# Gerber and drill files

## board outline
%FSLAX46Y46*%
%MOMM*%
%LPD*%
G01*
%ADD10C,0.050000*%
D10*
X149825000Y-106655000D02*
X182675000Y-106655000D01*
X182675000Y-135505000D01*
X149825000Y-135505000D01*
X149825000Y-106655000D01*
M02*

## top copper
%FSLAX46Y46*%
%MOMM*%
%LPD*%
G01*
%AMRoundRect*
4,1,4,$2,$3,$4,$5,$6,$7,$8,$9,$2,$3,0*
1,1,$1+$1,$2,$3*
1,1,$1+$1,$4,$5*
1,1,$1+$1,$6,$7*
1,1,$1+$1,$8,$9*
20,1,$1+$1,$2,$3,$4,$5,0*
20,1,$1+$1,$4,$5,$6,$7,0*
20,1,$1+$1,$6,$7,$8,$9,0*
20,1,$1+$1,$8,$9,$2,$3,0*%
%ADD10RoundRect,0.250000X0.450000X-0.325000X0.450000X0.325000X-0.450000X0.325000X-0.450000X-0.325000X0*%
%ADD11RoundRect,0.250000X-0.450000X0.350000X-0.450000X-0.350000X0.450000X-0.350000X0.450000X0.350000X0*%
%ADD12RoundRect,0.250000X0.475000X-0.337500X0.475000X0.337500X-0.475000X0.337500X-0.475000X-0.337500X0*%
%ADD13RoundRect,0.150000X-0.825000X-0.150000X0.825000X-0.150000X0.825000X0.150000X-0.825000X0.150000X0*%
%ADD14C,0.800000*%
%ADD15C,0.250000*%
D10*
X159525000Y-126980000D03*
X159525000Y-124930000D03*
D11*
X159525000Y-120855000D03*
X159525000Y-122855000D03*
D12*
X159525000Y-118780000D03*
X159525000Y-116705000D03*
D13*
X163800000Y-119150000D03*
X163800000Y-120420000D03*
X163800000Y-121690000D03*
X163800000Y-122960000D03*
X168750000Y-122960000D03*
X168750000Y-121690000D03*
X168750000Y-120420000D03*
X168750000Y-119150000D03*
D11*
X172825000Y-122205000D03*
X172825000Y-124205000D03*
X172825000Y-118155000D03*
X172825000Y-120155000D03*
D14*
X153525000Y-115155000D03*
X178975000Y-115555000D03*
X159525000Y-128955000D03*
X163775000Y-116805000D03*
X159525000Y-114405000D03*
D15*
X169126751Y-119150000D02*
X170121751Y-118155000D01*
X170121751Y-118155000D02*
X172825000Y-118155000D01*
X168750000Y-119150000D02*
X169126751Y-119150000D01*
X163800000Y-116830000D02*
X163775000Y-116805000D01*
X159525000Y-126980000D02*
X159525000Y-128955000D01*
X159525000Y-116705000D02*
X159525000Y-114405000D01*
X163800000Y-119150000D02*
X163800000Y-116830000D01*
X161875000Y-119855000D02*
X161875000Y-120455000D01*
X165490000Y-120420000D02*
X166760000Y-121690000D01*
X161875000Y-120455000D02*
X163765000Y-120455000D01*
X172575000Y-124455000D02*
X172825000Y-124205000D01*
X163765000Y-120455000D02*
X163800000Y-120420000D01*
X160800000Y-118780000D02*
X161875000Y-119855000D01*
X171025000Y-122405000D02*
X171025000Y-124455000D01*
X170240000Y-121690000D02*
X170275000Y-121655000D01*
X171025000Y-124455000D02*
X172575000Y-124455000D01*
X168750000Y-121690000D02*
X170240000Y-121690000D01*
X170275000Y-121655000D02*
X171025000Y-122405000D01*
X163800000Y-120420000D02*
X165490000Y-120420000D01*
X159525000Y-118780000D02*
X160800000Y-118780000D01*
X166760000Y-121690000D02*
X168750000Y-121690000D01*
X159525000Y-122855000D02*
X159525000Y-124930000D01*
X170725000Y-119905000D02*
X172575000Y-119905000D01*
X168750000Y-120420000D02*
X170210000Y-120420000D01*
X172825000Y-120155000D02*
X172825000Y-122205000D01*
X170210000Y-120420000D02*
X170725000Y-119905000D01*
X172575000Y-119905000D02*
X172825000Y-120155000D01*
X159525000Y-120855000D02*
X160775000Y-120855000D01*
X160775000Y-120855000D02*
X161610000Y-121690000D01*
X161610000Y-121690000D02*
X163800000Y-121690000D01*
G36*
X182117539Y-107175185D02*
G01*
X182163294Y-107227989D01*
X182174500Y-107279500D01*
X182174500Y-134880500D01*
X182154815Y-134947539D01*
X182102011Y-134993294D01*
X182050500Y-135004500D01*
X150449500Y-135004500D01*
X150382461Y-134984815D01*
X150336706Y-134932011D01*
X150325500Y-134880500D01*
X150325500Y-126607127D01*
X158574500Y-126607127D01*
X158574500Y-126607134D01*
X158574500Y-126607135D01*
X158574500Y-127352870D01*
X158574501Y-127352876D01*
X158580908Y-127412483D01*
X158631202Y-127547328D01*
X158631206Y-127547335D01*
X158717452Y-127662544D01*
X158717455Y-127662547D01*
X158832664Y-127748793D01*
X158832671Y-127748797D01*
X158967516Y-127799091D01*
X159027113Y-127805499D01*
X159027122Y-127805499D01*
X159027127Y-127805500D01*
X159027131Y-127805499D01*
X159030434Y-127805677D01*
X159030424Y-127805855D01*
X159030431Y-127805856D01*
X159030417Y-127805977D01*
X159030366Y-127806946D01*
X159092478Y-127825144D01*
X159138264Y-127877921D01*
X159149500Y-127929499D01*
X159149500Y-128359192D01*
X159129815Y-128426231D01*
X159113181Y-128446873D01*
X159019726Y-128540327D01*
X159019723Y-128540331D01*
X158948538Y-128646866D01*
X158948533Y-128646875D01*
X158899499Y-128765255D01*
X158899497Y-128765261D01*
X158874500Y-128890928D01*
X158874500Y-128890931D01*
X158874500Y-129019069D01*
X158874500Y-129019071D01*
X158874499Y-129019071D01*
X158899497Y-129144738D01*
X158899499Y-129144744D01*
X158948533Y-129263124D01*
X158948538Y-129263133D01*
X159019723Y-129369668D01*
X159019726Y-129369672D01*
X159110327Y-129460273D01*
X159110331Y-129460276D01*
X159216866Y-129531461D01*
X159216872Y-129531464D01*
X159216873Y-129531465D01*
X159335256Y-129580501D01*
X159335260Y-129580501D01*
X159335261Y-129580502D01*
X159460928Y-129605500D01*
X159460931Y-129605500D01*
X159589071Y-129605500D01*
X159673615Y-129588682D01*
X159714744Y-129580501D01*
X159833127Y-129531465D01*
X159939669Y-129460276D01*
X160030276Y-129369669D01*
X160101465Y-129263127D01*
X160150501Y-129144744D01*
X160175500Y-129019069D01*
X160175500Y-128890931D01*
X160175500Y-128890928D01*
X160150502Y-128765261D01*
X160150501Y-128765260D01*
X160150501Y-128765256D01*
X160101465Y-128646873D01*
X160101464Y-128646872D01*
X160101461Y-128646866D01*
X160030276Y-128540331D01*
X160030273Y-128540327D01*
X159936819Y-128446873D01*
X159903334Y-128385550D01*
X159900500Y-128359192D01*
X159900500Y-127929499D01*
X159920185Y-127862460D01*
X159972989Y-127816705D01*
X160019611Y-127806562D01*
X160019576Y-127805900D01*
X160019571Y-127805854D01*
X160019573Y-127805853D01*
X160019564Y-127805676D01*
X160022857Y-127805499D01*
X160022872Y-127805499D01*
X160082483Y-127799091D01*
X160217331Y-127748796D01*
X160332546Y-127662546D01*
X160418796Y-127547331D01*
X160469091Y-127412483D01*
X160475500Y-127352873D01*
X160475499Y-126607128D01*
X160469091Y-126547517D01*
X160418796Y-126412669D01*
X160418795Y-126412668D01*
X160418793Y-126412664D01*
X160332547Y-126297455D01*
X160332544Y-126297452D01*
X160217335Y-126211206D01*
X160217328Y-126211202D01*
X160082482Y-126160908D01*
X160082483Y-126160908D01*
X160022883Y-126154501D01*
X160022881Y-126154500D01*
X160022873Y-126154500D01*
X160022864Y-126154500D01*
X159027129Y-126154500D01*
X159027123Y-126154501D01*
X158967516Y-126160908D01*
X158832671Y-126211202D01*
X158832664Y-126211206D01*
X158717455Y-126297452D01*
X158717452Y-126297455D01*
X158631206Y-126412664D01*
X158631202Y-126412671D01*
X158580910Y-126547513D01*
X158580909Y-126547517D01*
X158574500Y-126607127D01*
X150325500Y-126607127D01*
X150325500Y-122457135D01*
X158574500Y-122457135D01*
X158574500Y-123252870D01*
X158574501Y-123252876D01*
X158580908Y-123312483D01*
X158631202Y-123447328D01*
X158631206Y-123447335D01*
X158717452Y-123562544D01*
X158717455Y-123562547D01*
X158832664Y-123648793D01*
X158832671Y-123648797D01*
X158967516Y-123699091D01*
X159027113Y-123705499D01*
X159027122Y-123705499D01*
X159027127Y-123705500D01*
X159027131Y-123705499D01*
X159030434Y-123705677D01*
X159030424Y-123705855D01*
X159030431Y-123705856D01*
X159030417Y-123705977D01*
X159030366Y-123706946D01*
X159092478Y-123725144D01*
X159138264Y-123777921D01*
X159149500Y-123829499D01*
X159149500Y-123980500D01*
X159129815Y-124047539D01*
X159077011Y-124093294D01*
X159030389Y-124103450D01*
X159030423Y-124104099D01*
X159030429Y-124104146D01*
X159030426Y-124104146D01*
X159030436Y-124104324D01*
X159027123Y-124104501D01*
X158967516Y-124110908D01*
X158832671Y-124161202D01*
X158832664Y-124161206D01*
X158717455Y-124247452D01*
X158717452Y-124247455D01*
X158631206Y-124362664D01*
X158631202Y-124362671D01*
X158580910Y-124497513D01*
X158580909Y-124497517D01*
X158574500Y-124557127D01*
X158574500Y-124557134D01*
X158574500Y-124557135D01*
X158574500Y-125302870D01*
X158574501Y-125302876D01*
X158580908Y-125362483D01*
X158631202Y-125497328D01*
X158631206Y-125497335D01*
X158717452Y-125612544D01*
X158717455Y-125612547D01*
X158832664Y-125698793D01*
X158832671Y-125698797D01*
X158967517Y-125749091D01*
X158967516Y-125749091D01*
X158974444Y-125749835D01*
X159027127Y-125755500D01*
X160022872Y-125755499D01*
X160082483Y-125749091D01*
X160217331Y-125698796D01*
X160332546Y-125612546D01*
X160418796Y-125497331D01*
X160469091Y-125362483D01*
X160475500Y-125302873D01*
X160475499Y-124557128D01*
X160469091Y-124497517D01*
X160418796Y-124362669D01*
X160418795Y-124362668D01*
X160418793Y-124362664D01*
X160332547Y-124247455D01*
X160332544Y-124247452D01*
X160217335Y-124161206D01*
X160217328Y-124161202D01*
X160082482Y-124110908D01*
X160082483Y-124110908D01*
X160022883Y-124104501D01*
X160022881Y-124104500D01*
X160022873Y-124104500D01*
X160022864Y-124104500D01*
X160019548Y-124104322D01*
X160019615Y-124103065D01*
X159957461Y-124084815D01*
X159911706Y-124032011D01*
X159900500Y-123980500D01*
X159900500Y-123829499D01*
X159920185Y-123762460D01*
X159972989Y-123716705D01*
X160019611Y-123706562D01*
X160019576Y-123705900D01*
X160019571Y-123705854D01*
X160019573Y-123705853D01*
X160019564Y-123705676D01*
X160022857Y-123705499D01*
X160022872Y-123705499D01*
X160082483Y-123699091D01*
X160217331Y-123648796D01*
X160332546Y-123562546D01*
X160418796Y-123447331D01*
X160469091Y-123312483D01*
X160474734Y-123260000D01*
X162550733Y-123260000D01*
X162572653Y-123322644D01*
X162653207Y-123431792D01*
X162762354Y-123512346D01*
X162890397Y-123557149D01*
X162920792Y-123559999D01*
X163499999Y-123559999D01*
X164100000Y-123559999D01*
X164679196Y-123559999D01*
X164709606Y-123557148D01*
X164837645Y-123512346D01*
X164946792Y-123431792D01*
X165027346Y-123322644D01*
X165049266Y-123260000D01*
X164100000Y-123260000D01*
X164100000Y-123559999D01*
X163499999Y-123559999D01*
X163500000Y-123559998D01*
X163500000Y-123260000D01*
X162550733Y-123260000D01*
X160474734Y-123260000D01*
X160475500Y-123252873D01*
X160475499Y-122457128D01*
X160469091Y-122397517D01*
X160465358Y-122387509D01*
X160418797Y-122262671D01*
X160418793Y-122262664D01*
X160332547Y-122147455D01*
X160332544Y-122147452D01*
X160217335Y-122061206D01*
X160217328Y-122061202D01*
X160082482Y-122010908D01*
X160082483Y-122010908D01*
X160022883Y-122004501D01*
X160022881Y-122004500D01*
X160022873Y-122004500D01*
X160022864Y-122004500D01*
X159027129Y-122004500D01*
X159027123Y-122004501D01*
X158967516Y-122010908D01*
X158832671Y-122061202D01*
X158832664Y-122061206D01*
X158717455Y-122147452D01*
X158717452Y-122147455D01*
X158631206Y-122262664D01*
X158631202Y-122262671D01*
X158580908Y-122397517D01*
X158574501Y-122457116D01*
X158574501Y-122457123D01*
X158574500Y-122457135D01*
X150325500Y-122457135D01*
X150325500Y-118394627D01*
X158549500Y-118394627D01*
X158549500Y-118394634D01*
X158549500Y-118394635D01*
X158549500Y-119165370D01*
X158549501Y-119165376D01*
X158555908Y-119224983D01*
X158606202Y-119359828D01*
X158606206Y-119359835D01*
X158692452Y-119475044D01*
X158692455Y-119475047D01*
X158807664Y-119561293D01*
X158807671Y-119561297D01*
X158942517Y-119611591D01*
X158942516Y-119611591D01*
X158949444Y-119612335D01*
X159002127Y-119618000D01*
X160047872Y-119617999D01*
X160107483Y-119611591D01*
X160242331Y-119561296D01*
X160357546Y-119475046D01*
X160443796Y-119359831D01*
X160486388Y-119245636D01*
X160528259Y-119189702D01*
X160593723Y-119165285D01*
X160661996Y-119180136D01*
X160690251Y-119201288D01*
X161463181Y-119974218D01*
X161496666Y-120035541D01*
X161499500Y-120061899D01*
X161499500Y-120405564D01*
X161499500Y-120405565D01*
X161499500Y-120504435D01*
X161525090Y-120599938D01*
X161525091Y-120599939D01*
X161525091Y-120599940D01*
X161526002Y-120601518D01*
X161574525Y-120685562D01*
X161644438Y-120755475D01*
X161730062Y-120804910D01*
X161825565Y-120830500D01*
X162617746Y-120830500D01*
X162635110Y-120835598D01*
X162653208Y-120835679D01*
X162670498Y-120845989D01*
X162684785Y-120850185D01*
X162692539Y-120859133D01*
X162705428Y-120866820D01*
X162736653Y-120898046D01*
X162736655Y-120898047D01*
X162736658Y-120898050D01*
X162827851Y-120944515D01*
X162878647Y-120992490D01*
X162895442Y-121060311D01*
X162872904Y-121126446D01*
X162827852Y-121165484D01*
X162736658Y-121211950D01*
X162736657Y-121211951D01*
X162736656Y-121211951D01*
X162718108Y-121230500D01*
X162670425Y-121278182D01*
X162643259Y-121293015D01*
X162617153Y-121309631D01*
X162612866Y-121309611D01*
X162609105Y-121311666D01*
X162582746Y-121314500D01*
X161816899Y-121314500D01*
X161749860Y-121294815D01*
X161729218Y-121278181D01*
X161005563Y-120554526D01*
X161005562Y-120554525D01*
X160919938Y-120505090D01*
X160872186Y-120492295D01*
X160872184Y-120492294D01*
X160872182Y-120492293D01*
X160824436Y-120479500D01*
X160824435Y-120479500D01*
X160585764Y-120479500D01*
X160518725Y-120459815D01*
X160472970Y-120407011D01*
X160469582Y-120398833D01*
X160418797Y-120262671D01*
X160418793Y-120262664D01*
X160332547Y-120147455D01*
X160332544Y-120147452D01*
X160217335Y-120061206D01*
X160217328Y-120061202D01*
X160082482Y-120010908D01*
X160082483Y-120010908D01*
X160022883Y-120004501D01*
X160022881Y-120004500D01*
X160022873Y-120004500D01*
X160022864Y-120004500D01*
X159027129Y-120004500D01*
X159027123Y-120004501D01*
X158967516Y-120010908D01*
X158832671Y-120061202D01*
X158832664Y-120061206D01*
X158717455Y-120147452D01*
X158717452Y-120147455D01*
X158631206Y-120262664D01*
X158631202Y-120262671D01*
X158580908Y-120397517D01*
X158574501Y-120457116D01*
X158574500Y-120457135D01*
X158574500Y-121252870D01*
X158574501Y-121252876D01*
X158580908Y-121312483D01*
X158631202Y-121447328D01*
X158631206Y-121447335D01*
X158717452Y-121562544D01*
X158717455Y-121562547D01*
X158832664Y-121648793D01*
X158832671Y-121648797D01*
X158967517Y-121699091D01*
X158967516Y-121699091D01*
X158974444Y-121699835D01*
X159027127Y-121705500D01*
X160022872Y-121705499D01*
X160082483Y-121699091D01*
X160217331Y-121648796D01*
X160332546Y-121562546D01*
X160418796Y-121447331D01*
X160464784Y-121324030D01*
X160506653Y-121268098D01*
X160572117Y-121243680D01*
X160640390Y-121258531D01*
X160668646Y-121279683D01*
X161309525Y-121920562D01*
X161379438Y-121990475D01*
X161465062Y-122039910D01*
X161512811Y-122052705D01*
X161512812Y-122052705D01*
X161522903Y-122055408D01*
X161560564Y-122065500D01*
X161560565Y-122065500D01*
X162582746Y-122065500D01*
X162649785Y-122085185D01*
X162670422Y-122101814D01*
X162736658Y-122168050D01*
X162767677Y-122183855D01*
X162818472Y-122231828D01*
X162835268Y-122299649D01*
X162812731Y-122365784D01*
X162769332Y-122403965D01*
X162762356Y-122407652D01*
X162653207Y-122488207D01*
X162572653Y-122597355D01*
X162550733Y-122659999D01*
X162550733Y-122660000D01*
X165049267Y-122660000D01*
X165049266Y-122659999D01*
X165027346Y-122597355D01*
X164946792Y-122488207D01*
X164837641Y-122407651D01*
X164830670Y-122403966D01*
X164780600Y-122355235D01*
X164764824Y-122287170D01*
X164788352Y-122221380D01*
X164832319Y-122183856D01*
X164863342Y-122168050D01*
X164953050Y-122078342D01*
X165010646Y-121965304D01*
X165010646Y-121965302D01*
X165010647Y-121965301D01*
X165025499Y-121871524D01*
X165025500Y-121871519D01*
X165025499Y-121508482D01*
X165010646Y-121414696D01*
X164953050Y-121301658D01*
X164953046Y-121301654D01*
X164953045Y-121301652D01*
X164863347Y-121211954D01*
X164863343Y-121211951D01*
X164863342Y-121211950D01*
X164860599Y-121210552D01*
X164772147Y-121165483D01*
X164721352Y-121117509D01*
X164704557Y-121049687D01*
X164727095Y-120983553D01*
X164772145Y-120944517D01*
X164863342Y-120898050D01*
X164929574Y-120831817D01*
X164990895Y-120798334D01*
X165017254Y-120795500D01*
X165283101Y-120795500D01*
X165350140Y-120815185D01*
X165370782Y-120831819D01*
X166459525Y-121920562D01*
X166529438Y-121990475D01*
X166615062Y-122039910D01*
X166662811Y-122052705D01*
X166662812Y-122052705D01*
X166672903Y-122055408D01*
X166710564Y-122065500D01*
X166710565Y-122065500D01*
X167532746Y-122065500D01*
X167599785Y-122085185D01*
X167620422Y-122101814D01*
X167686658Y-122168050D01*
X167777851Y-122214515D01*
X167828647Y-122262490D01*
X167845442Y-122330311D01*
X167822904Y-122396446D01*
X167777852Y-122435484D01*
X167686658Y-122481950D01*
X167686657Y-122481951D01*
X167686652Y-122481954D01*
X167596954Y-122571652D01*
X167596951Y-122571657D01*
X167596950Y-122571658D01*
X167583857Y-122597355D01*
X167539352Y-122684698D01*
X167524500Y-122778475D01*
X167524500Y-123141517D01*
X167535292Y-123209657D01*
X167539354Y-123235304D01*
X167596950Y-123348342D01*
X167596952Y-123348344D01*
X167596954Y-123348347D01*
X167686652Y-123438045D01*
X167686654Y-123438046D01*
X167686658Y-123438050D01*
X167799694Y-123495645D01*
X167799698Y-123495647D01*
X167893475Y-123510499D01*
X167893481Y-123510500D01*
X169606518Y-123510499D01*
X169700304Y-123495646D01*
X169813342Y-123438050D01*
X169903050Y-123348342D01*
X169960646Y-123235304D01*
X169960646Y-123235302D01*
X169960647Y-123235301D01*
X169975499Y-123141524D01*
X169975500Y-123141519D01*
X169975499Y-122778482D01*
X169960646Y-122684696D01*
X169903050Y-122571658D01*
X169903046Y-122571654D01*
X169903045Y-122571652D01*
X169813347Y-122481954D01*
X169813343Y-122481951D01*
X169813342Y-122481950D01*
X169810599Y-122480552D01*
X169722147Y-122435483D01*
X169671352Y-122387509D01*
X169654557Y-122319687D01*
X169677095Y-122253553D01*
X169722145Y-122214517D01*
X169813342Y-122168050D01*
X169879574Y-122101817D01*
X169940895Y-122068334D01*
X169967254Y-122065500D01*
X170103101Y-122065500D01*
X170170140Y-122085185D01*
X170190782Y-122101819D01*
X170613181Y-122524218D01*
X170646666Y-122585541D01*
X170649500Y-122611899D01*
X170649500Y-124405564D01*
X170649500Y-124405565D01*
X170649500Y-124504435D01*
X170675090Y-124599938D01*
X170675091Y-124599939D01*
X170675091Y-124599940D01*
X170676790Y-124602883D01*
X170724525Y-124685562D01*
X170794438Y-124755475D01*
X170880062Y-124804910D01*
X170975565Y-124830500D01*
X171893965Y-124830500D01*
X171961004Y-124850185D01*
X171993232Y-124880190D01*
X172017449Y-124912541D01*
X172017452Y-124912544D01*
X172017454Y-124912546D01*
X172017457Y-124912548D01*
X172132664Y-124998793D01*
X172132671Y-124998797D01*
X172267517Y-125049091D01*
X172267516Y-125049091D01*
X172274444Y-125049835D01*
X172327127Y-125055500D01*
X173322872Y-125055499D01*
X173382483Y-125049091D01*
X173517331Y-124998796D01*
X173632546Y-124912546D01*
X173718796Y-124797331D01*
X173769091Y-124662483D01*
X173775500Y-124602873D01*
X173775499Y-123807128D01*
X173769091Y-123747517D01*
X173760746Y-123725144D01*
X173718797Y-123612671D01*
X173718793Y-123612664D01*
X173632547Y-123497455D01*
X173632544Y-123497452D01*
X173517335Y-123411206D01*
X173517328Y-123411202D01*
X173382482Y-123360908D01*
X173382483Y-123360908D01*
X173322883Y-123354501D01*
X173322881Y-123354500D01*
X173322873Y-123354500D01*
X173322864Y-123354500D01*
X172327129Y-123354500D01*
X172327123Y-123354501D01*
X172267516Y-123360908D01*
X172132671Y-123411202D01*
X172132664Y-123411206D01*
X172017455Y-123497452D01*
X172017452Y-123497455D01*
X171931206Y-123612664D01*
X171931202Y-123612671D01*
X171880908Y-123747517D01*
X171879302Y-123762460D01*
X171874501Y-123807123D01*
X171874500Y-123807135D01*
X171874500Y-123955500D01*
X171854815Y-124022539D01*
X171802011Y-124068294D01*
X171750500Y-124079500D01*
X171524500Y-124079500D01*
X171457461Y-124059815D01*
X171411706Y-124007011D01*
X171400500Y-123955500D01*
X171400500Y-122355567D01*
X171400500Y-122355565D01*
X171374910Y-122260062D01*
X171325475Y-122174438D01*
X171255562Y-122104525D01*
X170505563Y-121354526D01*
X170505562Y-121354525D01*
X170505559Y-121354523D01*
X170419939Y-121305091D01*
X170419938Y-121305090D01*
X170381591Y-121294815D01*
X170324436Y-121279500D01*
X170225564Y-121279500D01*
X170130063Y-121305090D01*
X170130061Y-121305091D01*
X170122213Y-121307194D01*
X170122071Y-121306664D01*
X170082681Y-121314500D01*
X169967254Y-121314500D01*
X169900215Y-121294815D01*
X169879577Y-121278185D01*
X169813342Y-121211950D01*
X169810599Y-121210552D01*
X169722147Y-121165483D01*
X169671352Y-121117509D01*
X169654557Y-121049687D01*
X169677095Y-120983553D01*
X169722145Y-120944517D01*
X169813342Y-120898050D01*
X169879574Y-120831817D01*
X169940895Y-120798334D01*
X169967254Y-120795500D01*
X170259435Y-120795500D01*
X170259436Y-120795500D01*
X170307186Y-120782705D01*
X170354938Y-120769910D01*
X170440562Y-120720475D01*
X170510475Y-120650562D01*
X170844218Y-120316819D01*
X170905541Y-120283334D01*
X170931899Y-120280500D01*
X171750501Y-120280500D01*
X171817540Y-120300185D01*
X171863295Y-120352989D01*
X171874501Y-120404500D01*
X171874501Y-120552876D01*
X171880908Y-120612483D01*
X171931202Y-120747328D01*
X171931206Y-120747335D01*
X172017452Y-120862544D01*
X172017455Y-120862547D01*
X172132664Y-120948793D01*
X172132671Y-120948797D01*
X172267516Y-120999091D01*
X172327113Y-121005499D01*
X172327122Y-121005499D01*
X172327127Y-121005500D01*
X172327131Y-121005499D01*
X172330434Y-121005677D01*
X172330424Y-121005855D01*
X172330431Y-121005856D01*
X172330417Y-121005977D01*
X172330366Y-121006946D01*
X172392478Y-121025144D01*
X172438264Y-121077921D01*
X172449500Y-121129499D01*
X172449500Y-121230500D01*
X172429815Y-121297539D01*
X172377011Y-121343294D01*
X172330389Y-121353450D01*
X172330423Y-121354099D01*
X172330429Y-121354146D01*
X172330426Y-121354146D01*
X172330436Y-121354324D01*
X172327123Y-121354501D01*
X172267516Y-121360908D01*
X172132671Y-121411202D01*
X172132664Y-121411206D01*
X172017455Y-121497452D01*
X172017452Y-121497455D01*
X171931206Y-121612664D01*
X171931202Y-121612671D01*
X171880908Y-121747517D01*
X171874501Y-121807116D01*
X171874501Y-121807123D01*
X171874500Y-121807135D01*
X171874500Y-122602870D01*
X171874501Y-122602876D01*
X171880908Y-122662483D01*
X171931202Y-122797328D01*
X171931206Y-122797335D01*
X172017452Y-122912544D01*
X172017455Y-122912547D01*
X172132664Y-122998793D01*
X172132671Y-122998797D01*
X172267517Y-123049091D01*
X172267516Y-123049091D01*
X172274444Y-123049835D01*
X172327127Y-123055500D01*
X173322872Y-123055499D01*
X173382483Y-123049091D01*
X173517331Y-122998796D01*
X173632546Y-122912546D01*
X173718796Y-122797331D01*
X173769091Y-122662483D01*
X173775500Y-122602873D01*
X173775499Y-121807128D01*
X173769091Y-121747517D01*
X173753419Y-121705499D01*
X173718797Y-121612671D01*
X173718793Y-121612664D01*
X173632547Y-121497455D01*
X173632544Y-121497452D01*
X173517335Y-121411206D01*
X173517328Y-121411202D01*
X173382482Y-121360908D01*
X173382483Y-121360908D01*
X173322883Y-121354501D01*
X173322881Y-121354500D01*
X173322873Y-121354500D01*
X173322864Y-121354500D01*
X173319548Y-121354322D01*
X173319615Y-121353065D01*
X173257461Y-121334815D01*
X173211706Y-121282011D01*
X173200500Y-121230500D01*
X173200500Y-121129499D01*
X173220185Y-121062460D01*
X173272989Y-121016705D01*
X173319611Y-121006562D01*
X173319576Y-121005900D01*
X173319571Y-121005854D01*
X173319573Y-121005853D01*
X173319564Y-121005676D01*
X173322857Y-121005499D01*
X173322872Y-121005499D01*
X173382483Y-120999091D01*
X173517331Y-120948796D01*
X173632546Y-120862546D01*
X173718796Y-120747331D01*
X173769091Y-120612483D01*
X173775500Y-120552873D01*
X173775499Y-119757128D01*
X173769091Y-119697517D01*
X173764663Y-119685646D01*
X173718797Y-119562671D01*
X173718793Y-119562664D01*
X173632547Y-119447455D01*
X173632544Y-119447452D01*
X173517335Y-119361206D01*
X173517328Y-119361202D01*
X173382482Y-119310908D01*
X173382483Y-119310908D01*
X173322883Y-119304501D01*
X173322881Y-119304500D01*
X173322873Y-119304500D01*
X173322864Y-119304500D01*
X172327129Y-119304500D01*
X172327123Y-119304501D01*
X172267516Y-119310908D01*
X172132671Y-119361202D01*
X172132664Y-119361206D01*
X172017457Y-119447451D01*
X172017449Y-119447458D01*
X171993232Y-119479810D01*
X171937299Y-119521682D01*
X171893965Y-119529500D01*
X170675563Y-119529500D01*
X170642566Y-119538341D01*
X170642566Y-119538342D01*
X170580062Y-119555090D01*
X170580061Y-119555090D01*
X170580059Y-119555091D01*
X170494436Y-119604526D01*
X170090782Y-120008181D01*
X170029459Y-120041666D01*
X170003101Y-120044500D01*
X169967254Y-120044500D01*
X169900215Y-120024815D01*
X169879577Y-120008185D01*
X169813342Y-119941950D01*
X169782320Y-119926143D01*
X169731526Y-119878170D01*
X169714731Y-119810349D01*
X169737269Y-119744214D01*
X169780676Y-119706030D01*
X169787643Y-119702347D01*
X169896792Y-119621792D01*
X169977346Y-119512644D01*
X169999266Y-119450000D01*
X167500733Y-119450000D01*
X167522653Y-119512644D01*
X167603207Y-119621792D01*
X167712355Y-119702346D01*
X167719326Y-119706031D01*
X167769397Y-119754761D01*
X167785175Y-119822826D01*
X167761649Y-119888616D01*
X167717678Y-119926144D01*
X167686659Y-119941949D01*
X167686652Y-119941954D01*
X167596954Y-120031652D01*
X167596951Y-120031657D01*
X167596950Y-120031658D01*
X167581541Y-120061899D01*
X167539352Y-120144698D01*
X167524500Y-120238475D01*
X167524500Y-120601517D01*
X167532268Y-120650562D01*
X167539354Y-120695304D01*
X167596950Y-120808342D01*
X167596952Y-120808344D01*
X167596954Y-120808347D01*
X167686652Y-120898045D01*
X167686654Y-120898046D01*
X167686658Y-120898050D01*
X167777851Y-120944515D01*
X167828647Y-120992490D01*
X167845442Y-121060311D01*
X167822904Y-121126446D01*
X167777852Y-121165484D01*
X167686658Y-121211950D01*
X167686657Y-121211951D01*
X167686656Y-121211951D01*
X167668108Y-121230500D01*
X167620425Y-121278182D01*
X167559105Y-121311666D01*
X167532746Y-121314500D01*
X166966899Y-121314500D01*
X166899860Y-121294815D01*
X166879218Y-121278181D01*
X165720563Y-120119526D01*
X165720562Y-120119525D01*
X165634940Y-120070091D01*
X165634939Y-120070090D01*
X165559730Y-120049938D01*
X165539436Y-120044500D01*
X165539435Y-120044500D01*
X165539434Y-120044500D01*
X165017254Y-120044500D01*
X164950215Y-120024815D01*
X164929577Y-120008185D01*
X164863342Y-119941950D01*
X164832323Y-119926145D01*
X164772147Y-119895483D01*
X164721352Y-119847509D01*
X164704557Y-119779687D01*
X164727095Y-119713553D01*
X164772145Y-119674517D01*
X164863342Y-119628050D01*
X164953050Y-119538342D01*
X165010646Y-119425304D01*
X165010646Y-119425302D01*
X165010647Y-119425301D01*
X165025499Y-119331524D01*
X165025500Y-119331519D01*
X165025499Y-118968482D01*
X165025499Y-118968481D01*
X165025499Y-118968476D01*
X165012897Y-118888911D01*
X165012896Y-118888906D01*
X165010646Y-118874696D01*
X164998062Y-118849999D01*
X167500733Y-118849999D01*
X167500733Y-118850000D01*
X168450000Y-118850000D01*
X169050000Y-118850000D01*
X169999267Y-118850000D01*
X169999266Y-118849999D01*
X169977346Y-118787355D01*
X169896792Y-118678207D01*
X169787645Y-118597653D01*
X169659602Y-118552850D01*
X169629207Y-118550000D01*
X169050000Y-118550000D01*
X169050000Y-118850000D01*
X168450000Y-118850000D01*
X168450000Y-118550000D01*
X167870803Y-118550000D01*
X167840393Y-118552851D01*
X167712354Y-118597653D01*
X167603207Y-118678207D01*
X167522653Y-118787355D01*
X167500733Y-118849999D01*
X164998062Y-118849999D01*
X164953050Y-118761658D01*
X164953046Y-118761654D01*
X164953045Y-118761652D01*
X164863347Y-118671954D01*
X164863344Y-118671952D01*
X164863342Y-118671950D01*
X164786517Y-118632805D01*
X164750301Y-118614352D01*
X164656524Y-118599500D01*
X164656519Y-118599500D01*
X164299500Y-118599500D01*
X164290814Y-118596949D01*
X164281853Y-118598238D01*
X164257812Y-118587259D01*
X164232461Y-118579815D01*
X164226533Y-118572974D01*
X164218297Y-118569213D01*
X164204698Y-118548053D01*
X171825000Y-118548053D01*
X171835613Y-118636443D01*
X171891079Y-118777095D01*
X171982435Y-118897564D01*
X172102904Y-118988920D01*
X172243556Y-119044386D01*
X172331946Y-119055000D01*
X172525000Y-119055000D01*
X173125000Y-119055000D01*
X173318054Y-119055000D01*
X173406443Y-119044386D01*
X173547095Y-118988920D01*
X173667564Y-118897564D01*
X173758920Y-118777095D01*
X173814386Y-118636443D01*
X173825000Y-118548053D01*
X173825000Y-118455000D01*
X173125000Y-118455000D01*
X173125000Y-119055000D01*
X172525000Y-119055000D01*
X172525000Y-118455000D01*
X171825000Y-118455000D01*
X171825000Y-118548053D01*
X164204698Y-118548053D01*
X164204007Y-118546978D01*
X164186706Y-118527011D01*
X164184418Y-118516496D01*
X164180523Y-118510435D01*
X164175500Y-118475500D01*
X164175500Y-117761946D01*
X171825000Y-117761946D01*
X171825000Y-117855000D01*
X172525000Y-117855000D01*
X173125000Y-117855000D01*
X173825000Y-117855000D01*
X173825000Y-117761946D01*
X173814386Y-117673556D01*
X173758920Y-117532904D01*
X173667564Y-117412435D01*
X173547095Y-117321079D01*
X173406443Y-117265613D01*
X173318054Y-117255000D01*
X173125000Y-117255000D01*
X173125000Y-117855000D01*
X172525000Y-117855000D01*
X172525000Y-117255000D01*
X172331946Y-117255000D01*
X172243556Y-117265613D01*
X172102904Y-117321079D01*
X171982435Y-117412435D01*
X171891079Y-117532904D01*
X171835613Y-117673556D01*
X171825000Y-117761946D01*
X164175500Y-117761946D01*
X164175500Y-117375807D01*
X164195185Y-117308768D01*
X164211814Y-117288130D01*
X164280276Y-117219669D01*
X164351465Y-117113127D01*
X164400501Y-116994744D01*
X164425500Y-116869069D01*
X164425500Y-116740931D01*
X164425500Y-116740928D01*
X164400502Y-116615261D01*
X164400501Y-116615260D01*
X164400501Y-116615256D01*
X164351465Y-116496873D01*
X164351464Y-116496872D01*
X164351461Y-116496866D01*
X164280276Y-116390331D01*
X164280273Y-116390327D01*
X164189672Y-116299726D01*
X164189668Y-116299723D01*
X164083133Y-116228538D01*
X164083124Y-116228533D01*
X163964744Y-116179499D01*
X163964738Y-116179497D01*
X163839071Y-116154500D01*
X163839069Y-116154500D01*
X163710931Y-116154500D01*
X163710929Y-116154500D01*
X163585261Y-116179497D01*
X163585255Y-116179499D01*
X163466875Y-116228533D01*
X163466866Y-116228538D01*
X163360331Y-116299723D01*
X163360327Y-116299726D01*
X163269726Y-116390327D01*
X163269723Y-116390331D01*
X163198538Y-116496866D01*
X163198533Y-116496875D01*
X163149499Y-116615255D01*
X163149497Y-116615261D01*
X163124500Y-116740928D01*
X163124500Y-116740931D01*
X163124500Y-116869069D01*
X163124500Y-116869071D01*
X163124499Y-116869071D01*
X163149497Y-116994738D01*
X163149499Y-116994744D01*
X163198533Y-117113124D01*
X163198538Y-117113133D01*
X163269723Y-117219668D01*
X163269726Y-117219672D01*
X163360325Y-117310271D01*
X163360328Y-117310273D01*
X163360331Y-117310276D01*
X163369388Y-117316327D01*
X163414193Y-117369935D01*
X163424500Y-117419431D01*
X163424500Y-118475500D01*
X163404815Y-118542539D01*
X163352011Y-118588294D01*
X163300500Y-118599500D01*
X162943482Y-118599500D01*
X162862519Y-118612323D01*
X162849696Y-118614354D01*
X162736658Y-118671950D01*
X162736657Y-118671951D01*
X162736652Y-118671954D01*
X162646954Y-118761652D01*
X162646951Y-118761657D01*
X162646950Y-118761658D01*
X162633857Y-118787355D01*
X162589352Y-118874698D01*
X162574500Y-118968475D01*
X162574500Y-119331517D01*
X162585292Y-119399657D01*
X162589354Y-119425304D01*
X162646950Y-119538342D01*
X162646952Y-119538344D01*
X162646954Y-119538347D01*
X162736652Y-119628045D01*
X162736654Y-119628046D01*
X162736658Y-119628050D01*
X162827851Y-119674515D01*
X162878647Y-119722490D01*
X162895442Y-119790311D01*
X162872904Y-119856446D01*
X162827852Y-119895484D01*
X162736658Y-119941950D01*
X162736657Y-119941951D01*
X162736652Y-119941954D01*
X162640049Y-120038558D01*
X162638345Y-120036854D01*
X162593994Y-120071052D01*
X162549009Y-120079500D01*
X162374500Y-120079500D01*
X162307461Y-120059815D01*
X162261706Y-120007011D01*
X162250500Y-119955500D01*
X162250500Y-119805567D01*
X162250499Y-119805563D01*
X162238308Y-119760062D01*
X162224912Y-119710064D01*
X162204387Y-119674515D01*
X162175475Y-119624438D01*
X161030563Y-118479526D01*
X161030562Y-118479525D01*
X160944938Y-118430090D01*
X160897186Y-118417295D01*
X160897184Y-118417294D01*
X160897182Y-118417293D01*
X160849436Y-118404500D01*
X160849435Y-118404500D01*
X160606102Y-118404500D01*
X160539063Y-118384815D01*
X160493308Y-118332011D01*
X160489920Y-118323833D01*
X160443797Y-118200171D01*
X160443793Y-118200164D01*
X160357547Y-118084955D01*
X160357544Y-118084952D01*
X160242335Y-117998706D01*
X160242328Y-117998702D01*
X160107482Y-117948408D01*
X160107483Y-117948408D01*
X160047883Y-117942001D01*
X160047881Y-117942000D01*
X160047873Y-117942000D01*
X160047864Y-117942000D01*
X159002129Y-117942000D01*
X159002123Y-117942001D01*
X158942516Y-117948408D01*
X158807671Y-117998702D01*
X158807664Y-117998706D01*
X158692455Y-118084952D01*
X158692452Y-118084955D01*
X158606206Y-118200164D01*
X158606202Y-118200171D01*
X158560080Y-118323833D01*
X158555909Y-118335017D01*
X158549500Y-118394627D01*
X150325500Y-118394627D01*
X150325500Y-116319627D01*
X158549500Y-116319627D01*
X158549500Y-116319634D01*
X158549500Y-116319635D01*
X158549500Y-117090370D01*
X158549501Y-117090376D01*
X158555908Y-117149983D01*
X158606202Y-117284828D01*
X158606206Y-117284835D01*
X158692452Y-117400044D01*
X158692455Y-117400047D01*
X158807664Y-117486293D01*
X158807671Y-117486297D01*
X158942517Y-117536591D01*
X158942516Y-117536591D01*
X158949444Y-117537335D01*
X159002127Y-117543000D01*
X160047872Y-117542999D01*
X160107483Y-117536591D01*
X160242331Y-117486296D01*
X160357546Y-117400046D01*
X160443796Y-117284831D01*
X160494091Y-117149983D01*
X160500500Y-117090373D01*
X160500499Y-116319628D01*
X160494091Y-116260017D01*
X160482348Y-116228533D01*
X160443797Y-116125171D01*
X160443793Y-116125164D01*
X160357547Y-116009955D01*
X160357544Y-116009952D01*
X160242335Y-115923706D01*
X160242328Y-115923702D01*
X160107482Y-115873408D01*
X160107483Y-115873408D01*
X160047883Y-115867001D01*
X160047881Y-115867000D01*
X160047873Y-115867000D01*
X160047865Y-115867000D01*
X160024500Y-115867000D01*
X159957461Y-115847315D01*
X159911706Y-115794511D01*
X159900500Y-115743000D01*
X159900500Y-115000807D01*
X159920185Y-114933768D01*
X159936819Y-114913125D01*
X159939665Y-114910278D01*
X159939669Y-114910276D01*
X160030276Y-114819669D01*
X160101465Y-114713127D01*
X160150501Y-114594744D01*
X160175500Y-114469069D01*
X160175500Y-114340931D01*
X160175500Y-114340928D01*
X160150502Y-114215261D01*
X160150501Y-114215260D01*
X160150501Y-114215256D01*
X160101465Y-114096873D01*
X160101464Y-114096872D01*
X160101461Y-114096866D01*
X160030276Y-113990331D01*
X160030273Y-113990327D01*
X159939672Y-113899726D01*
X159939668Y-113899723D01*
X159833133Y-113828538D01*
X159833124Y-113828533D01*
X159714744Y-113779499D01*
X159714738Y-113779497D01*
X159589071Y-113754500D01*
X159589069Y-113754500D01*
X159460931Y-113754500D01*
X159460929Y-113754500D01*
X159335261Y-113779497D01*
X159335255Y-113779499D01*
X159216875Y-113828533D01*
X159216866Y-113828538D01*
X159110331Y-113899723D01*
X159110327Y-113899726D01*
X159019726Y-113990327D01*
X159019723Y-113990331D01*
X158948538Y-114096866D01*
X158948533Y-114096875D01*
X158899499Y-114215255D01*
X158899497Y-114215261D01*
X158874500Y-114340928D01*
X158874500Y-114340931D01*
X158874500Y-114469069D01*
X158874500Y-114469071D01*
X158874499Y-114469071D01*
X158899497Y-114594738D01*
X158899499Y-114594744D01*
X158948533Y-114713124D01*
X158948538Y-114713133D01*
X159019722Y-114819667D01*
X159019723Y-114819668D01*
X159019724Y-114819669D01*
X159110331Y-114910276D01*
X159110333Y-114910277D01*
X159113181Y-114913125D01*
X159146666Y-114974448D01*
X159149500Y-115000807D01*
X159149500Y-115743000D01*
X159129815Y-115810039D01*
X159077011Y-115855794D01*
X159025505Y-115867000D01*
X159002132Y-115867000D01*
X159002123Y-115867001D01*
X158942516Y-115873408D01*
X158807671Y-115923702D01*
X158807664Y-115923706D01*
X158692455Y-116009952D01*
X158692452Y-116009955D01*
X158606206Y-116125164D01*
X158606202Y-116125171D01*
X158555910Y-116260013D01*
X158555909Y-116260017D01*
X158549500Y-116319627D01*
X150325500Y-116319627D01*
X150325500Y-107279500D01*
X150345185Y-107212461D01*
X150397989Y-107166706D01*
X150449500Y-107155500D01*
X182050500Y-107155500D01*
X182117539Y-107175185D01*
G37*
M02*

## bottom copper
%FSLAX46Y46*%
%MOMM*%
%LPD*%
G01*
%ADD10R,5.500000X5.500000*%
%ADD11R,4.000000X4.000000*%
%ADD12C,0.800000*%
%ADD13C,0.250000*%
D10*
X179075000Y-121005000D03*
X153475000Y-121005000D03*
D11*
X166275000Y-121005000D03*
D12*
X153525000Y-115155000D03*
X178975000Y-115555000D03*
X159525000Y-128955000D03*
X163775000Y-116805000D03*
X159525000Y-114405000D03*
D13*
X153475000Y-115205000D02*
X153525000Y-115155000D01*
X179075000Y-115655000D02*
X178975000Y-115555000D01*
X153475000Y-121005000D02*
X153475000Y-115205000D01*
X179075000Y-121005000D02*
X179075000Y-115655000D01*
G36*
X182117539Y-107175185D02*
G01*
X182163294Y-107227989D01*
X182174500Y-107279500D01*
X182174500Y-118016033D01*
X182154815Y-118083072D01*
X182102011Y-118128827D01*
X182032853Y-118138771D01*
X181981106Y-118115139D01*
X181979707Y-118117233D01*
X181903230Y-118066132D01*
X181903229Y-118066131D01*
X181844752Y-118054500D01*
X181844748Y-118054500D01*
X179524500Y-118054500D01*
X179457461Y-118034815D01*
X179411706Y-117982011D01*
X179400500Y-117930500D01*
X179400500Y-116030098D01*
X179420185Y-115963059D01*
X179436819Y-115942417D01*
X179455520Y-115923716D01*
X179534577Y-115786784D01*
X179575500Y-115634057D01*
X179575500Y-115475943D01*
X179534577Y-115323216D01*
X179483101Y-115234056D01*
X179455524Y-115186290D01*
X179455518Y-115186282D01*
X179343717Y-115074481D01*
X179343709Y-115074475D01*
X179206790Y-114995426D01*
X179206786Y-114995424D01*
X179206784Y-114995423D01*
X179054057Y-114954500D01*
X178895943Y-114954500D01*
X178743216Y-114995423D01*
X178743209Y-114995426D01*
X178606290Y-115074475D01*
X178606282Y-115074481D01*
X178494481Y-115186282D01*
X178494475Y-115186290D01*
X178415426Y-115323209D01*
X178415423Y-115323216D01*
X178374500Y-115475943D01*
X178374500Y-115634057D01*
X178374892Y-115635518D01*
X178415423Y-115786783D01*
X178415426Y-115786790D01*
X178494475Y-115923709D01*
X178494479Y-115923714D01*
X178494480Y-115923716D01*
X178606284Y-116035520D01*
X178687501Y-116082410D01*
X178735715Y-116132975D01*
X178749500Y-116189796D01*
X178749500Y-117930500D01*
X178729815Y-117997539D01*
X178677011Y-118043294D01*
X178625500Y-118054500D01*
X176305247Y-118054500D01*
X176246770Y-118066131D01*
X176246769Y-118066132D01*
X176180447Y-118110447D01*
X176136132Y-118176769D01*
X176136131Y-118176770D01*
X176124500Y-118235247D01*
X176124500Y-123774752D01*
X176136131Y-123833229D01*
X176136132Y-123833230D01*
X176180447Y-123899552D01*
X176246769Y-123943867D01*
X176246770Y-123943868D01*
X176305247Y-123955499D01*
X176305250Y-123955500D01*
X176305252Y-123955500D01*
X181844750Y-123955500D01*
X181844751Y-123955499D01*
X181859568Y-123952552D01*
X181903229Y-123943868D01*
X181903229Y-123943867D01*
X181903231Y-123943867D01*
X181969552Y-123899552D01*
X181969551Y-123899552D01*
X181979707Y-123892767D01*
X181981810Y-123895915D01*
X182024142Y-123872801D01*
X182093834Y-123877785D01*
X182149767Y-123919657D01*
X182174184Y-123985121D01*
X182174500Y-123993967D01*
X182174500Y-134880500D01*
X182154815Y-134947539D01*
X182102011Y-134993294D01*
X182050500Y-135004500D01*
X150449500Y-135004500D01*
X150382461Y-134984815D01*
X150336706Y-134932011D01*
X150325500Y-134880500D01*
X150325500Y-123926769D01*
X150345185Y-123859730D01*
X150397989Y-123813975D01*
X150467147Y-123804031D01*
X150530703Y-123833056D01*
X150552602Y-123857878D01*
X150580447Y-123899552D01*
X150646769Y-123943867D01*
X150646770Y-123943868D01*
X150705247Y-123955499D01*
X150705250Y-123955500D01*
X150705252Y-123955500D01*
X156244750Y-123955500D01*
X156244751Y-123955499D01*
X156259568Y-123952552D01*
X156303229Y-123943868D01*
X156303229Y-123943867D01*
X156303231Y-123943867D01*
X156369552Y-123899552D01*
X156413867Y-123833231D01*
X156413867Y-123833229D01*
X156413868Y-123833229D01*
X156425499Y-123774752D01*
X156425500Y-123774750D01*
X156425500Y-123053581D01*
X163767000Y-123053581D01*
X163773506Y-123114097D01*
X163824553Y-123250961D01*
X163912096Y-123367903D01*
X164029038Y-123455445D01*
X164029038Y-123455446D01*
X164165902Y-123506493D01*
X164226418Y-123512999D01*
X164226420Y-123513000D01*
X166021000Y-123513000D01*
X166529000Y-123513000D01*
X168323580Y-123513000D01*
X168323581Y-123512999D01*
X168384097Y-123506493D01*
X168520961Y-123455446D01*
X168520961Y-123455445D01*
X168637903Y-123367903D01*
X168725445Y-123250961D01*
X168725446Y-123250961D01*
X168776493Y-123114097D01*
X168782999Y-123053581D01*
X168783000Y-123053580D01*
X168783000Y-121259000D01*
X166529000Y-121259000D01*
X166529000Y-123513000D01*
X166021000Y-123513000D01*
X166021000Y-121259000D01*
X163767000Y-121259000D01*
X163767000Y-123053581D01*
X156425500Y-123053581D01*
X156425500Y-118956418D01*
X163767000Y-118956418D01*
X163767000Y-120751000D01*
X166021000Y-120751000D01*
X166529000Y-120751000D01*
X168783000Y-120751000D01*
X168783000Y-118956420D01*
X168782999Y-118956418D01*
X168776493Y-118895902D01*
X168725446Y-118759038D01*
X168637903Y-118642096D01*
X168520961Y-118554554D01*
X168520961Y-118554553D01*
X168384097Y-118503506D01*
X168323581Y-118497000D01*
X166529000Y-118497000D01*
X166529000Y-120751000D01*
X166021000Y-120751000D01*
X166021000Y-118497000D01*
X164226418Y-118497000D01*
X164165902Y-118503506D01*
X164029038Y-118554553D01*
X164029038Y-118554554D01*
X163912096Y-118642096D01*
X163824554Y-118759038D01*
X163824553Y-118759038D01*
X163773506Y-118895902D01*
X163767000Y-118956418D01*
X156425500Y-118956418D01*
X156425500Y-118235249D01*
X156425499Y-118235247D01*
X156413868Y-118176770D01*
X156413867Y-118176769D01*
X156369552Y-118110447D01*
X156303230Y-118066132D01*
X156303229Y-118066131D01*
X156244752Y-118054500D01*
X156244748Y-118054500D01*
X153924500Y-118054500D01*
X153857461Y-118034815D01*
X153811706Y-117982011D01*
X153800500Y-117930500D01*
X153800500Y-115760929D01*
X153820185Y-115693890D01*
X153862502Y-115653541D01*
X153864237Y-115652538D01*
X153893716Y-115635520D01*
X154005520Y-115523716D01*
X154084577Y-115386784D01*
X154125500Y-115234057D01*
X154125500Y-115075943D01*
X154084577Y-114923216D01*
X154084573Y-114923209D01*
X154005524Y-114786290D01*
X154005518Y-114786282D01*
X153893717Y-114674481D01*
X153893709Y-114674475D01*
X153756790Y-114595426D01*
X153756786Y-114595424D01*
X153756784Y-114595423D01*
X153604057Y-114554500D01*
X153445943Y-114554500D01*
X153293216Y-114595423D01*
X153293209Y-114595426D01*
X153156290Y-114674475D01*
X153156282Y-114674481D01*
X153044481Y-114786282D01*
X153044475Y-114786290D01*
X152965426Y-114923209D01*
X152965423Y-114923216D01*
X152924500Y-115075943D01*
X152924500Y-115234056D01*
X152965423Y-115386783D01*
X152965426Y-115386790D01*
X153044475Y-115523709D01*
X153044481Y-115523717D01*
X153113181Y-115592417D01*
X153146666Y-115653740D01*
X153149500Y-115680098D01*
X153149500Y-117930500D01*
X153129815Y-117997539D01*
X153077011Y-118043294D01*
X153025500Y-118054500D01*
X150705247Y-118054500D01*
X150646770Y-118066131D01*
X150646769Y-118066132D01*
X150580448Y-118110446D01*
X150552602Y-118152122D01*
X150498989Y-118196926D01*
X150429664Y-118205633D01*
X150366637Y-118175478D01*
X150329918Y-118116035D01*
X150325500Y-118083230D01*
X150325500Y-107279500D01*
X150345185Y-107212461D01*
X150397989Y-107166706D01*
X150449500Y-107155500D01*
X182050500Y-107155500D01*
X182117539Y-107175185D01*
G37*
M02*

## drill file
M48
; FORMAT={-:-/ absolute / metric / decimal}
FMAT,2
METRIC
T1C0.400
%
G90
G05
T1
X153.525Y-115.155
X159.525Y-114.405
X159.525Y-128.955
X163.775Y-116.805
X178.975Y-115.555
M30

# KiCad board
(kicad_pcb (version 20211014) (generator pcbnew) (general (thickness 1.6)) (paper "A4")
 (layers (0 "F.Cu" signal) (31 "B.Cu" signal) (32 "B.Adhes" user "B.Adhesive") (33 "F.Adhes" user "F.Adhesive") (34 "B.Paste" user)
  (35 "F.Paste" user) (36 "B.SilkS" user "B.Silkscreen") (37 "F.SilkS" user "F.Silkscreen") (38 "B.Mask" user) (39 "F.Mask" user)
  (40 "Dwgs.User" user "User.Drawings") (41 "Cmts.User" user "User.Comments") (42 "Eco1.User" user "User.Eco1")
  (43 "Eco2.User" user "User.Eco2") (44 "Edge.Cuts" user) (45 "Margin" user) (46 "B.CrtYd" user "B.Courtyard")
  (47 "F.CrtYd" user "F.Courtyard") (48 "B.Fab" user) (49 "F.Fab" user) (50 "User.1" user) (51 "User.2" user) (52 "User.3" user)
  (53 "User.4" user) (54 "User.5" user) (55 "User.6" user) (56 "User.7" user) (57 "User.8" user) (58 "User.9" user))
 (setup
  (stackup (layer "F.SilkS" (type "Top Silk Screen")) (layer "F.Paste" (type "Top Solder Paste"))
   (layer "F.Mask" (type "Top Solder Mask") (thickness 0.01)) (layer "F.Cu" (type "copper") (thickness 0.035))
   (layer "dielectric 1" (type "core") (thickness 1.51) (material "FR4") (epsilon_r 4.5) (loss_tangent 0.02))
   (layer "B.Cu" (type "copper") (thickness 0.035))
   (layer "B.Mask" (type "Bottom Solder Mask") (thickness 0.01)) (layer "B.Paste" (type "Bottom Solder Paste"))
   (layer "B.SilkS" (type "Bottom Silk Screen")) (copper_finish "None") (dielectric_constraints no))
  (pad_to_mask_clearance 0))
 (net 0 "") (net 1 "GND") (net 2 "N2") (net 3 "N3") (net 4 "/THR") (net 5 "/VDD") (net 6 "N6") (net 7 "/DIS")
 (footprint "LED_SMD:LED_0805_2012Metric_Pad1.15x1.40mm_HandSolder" (layer "F.Cu") (at 159.525 125.955 90)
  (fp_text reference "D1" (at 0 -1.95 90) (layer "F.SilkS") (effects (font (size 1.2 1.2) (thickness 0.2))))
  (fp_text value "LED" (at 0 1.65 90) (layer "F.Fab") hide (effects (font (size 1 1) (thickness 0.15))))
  (pad "1" smd roundrect (at -1.025 0 90) (size 1.15 1.4) (layers "F.Cu" "F.Paste" "F.Mask") (roundrect_rratio 0.2173913043) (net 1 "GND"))
  (pad "2" smd roundrect (at 1.025 0 90) (size 1.15 1.4) (layers "F.Cu" "F.Paste" "F.Mask") (roundrect_rratio 0.2173913043) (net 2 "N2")))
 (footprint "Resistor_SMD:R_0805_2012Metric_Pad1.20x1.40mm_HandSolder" (layer "F.Cu") (at 159.525 121.855 -90)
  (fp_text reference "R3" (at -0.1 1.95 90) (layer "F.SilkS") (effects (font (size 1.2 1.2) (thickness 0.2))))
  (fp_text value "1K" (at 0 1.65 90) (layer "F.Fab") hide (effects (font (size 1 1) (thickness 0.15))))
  (pad "1" smd roundrect (at -1 0 270) (size 1.2 1.4) (layers "F.Cu" "F.Paste" "F.Mask") (roundrect_rratio 0.2083333333) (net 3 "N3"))
  (pad "2" smd roundrect (at 1 0 270) (size 1.2 1.4) (layers "F.Cu" "F.Paste" "F.Mask") (roundrect_rratio 0.2083333333) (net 2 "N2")))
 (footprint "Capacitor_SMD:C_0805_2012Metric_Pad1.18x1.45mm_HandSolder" (layer "F.Cu") (at 159.525 117.7425 90)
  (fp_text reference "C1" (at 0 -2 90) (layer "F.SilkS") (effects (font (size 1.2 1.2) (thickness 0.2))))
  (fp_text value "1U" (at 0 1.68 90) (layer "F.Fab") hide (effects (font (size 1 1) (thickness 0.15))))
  (pad "1" smd roundrect (at -1.0375 0 90) (size 1.175 1.45) (layers "F.Cu" "F.Paste" "F.Mask") (roundrect_rratio 0.2127659574)
   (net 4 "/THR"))
  (pad "2" smd roundrect (at 1.0375 0 90) (size 1.175 1.45) (layers "F.Cu" "F.Paste" "F.Mask") (roundrect_rratio 0.2127659574) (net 1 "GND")))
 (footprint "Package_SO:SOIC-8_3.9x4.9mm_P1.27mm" (layer "F.Cu") (at 166.275 121.055)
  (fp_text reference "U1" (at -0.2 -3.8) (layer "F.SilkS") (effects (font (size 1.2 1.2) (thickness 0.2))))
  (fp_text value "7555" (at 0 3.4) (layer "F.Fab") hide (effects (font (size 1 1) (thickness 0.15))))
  (pad "1" smd roundrect (at -2.475 -1.905) (size 1.95 0.6) (layers "F.Cu" "F.Paste" "F.Mask") (roundrect_rratio 0.25) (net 1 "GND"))
  (pad "2" smd roundrect (at -2.475 -0.635) (size 1.95 0.6) (layers "F.Cu" "F.Paste" "F.Mask") (roundrect_rratio 0.25) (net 4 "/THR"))
  (pad "3" smd roundrect (at -2.475 0.635) (size 1.95 0.6) (layers "F.Cu" "F.Paste" "F.Mask") (roundrect_rratio 0.25) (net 3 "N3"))
  (pad "4" smd roundrect (at -2.475 1.905) (size 1.95 0.6) (layers "F.Cu" "F.Paste" "F.Mask") (roundrect_rratio 0.25) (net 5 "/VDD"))
  (pad "5" smd roundrect (at 2.475 1.905) (size 1.95 0.6) (layers "F.Cu" "F.Paste" "F.Mask") (roundrect_rratio 0.25) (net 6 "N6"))
  (pad "6" smd roundrect (at 2.475 0.635) (size 1.95 0.6) (layers "F.Cu" "F.Paste" "F.Mask") (roundrect_rratio 0.25) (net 4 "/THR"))
  (pad "7" smd roundrect (at 2.475 -0.635) (size 1.95 0.6) (layers "F.Cu" "F.Paste" "F.Mask") (roundrect_rratio 0.25) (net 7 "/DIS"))
  (pad "8" smd roundrect (at 2.475 -1.905) (size 1.95 0.6) (layers "F.Cu" "F.Paste" "F.Mask") (roundrect_rratio 0.25) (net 5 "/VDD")))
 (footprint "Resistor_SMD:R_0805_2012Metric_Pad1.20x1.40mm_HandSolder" (layer "F.Cu") (at 172.825 123.205 -90)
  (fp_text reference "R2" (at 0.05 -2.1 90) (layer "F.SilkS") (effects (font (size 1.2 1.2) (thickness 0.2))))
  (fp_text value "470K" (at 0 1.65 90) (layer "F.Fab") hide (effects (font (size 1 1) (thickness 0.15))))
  (pad "1" smd roundrect (at -1 0 270) (size 1.2 1.4) (layers "F.Cu" "F.Paste" "F.Mask") (roundrect_rratio 0.2083333333) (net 7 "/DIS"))
  (pad "2" smd roundrect (at 1 0 270) (size 1.2 1.4) (layers "F.Cu" "F.Paste" "F.Mask") (roundrect_rratio 0.2083333333) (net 4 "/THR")))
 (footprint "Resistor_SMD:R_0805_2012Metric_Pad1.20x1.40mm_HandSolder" (layer "F.Cu") (at 172.825 119.155 -90)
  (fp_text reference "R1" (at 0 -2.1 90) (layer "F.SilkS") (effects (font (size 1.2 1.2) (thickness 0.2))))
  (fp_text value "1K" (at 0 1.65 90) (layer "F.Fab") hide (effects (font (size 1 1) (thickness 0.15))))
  (pad "1" smd roundrect (at -1 0 270) (size 1.2 1.4) (layers "F.Cu" "F.Paste" "F.Mask") (roundrect_rratio 0.2083333333) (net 5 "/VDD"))
  (pad "2" smd roundrect (at 1 0 270) (size 1.2 1.4) (layers "F.Cu" "F.Paste" "F.Mask") (roundrect_rratio 0.2083333333) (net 7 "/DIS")))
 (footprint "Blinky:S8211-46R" (layer "B.Cu") (at 166.275 121.005 180)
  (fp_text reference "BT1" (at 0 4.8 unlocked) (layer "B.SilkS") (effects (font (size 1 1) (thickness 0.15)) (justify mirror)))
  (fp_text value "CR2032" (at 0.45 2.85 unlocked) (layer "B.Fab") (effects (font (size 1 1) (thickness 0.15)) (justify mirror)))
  (pad "1" smd rect (at -12.8 0 180) (size 5.5 5.5) (layers "B.Cu" "B.Paste" "B.Mask") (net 5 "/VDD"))
  (pad "1" smd rect (at 12.8 0 180) (size 5.5 5.5) (layers "B.Cu" "B.Paste" "B.Mask") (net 5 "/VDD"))
  (pad "2" smd rect (at 0 0 180) (size 4 4) (layers "B.Cu" "B.Paste" "B.Mask") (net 1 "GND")))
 (gr_rect (start 149.825 106.655) (end 182.675 135.505) (layer "Edge.Cuts") (width 0.05) (fill none))
 (segment (start 169.126751 119.15) (end 170.121751 118.155) (width 0.25) (layer "F.Cu") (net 5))
 (segment (start 170.121751 118.155) (end 172.825 118.155) (width 0.25) (layer "F.Cu") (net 5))
 (segment (start 168.75 119.15) (end 169.126751 119.15) (width 0.25) (layer "F.Cu") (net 5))
 (via (at 153.525 115.155) (size 0.8) (drill 0.4) (layers "F.Cu" "B.Cu") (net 5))
 (via (at 178.975 115.555) (size 0.8) (drill 0.4) (layers "F.Cu" "B.Cu") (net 5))
 (segment (start 153.475 115.205) (end 153.525 115.155) (width 0.25) (layer "B.Cu") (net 5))
 (segment (start 179.075 115.655) (end 178.975 115.555) (width 0.25) (layer "B.Cu") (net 5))
 (segment (start 153.475 121.005) (end 153.475 115.205) (width 0.25) (layer "B.Cu") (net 5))
 (segment (start 179.075 121.005) (end 179.075 115.655) (width 0.25) (layer "B.Cu") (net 5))
 (segment (start 163.8 116.83) (end 163.775 116.805) (width 0.25) (layer "F.Cu") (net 1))
 (segment (start 159.525 126.98) (end 159.525 128.955) (width 0.25) (layer "F.Cu") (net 1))
 (segment (start 159.525 116.705) (end 159.525 114.405) (width 0.25) (layer "F.Cu") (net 1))
 (segment (start 163.8 119.15) (end 163.8 116.83) (width 0.25) (layer "F.Cu") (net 1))
 (via (at 159.525 128.955) (size 0.8) (drill 0.4) (layers "F.Cu" "B.Cu") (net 1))
 (via (at 163.775 116.805) (size 0.8) (drill 0.4) (layers "F.Cu" "B.Cu") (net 1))
 (via (at 159.525 114.405) (size 0.8) (drill 0.4) (layers "F.Cu" "B.Cu") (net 1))
 (segment (start 161.875 119.855) (end 161.875 120.455) (width 0.25) (layer "F.Cu") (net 4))
 (segment (start 165.49 120.42) (end 166.76 121.69) (width 0.25) (layer "F.Cu") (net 4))
 (segment (start 161.875 120.455) (end 163.765 120.455) (width 0.25) (layer "F.Cu") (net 4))
 (segment (start 172.575 124.455) (end 172.825 124.205) (width 0.25) (layer "F.Cu") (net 4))
 (segment (start 163.765 120.455) (end 163.8 120.42) (width 0.25) (layer "F.Cu") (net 4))
 (segment (start 160.8 118.78) (end 161.875 119.855) (width 0.25) (layer "F.Cu") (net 4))
 (segment (start 171.025 122.405) (end 171.025 124.455) (width 0.25) (layer "F.Cu") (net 4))
 (segment (start 170.24 121.69) (end 170.275 121.655) (width 0.25) (layer "F.Cu") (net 4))
 (segment (start 171.025 124.455) (end 172.575 124.455) (width 0.25) (layer "F.Cu") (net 4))
 (segment (start 168.75 121.69) (end 170.24 121.69) (width 0.25) (layer "F.Cu") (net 4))
 (segment (start 170.275 121.655) (end 171.025 122.405) (width 0.25) (layer "F.Cu") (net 4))
 (segment (start 163.8 120.42) (end 165.49 120.42) (width 0.25) (layer "F.Cu") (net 4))
 (segment (start 159.525 118.78) (end 160.8 118.78) (width 0.25) (layer "F.Cu") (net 4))
 (segment (start 166.76 121.69) (end 168.75 121.69) (width 0.25) (layer "F.Cu") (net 4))
 (segment (start 159.525 122.855) (end 159.525 124.93) (width 0.25) (layer "F.Cu") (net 2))
 (segment (start 170.725 119.905) (end 172.575 119.905) (width 0.25) (layer "F.Cu") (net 7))
 (segment (start 168.75 120.42) (end 170.21 120.42) (width 0.25) (layer "F.Cu") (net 7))
 (segment (start 172.825 120.155) (end 172.825 122.205) (width 0.25) (layer "F.Cu") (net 7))
 (segment (start 170.21 120.42) (end 170.725 119.905) (width 0.25) (layer "F.Cu") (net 7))
 (segment (start 172.575 119.905) (end 172.825 120.155) (width 0.25) (layer "F.Cu") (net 7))
 (segment (start 159.525 120.855) (end 160.775 120.855) (width 0.25) (layer "F.Cu") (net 3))
 (segment (start 160.775 120.855) (end 161.61 121.69) (width 0.25) (layer "F.Cu") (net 3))
 (segment (start 161.61 121.69) (end 163.8 121.69) (width 0.25) (layer "F.Cu") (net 3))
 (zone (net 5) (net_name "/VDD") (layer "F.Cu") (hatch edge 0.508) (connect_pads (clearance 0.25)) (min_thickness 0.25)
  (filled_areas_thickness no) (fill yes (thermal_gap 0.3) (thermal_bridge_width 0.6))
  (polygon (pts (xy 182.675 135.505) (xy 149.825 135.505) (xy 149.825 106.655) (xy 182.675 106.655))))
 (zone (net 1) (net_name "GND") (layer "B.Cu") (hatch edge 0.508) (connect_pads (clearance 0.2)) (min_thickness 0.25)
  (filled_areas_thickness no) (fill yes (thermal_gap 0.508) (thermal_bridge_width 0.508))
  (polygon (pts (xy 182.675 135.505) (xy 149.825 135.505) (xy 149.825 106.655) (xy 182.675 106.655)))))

